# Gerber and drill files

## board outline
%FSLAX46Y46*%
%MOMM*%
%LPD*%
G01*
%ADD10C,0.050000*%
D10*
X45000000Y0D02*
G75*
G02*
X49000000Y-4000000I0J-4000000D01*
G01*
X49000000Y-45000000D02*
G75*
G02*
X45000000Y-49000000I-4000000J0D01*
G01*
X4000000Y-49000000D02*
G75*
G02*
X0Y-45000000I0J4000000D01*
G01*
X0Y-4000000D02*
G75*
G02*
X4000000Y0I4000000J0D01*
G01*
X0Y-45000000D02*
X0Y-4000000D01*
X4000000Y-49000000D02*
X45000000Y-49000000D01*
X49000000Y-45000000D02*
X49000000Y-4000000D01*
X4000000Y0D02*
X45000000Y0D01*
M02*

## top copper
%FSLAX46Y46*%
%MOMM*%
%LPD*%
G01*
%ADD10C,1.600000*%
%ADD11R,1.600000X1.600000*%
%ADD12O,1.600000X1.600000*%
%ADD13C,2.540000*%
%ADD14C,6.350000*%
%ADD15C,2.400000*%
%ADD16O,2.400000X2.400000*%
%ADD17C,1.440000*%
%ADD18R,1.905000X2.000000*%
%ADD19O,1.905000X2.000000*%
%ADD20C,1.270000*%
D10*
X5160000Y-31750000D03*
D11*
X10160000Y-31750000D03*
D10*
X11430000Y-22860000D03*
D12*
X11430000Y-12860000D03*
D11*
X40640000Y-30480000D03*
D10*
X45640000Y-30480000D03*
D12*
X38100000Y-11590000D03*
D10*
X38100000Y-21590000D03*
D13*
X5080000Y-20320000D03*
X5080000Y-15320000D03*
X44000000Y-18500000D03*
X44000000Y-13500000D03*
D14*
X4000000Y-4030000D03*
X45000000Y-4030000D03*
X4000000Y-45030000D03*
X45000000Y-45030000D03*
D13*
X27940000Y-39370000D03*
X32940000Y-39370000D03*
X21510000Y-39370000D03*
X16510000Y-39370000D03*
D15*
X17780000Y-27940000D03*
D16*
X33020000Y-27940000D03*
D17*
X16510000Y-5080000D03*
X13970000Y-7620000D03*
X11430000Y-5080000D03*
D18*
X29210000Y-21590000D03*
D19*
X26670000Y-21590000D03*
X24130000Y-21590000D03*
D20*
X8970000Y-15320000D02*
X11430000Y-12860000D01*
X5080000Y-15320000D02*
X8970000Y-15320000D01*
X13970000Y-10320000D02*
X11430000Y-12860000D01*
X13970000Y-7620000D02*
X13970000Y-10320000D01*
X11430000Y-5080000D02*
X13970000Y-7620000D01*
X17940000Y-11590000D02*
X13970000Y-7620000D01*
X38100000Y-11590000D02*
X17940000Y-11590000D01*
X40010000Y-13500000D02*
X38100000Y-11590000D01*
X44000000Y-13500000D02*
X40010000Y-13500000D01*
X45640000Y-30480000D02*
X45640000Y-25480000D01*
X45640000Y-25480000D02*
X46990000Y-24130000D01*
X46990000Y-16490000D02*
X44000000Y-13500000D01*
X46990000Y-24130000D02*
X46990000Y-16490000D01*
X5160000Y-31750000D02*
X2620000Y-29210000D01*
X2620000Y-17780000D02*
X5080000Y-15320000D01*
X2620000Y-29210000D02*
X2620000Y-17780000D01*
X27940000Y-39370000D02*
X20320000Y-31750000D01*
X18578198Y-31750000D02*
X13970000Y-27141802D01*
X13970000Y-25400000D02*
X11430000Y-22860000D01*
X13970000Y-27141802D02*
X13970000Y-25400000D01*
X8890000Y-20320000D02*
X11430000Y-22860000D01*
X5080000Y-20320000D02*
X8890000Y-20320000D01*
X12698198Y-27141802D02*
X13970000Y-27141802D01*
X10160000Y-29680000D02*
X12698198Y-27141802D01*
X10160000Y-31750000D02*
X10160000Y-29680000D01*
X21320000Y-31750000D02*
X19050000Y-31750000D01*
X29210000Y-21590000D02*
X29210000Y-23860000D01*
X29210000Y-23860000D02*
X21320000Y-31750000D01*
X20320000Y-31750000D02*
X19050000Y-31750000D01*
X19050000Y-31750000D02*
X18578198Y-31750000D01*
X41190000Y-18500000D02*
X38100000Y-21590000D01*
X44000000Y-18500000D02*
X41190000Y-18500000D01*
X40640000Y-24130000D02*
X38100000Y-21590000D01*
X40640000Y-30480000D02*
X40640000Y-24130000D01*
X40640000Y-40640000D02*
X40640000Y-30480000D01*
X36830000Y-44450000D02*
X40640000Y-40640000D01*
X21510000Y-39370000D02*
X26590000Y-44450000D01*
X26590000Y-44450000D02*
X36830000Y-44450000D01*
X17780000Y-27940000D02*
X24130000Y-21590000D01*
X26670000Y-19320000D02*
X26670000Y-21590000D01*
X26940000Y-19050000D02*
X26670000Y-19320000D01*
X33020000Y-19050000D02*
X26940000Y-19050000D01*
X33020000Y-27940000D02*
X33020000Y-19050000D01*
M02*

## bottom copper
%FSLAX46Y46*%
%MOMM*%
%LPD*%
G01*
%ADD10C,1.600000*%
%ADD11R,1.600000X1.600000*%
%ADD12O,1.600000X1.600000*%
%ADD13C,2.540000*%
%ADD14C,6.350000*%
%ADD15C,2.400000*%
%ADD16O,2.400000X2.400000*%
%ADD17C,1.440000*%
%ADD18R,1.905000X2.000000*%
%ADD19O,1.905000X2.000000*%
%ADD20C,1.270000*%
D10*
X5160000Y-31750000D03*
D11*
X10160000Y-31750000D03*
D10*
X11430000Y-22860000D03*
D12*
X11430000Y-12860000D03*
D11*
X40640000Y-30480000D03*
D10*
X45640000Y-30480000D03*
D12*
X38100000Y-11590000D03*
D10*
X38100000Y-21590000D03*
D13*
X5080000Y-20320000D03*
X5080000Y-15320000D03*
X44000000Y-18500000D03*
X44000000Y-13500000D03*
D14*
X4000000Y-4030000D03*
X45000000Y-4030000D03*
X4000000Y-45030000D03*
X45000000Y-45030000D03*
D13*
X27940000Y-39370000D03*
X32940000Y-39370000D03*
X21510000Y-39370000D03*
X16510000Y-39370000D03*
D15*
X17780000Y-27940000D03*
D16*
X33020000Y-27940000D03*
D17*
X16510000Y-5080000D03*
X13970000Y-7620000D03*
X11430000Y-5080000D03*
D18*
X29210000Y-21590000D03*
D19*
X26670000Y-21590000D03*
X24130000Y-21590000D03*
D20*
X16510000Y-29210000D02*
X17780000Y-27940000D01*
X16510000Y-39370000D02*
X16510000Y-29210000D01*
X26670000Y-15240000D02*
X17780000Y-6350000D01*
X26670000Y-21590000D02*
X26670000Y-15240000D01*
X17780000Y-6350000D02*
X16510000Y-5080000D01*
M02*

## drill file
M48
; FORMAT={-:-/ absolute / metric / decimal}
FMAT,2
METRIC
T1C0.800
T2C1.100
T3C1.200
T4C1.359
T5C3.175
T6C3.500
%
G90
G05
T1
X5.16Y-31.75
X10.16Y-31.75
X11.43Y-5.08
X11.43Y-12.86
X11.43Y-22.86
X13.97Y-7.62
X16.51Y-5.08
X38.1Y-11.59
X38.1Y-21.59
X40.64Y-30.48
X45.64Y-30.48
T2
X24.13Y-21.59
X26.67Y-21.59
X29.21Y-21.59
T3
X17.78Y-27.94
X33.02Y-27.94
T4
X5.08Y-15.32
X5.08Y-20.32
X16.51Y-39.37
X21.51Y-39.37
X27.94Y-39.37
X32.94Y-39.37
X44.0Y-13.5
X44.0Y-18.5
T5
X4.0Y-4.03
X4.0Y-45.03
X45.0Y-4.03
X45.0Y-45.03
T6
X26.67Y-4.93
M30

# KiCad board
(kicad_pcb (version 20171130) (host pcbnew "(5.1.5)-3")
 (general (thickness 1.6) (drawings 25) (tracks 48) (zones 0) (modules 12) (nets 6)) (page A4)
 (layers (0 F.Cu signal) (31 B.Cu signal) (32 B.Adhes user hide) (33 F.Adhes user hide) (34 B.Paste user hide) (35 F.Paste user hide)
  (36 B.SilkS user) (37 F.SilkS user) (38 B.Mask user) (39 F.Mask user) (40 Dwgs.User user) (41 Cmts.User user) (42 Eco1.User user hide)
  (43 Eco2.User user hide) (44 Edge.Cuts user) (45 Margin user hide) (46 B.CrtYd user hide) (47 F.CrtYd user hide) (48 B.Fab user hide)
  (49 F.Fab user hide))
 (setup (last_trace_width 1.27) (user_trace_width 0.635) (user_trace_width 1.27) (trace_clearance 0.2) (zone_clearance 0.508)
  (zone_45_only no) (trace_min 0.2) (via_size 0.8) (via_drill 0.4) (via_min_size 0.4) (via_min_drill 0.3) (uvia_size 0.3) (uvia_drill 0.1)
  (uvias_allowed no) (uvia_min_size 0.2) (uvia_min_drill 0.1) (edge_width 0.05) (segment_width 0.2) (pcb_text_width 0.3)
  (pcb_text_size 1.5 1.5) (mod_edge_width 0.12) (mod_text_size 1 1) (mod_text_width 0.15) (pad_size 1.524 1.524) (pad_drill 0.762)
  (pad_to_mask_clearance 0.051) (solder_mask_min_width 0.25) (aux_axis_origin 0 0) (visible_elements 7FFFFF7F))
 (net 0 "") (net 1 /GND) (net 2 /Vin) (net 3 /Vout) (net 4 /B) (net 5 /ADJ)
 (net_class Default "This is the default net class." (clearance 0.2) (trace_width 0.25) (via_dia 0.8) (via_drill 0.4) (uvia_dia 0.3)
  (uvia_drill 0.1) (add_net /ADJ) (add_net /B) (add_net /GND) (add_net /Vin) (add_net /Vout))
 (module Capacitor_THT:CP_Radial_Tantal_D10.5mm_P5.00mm (layer F.Cu) (at 10.16 31.75 180)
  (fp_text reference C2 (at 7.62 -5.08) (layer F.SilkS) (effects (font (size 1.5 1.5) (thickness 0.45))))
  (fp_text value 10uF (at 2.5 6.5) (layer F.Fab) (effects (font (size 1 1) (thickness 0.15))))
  (pad 2 thru_hole circle (at 5 0 180) (size 1.6 1.6) (drill 0.8) (layers *.Cu *.Mask) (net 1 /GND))
  (pad 1 thru_hole rect (at 0 0 180) (size 1.6 1.6) (drill 0.8) (layers *.Cu *.Mask) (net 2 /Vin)))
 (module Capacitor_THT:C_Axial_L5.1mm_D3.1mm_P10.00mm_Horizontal (layer F.Cu) (at 11.43 22.86 90)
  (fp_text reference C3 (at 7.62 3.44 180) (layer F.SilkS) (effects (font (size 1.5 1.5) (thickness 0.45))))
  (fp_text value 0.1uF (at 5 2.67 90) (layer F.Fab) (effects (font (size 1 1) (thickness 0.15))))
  (pad 1 thru_hole circle (at 0 0 90) (size 1.6 1.6) (drill 0.8) (layers *.Cu *.Mask) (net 2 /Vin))
  (pad 2 thru_hole oval (at 10 0 90) (size 1.6 1.6) (drill 0.8) (layers *.Cu *.Mask) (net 1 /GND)))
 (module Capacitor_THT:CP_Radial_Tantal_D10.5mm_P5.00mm (layer F.Cu) (at 40.64 30.48)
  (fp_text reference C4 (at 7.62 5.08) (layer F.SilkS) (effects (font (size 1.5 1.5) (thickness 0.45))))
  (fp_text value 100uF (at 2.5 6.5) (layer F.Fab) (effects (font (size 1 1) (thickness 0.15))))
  (pad 1 thru_hole rect (at 0 0) (size 1.6 1.6) (drill 0.8) (layers *.Cu *.Mask) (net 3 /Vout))
  (pad 2 thru_hole circle (at 5 0) (size 1.6 1.6) (drill 0.8) (layers *.Cu *.Mask) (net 1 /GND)))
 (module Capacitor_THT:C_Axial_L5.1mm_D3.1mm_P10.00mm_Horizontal (layer F.Cu) (at 38.1 21.59 90)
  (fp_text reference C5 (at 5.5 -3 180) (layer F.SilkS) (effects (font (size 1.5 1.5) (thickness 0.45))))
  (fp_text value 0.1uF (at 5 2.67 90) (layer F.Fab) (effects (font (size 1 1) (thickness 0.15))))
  (pad 2 thru_hole oval (at 10 0 90) (size 1.6 1.6) (drill 0.8) (layers *.Cu *.Mask) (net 1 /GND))
  (pad 1 thru_hole circle (at 0 0 90) (size 1.6 1.6) (drill 0.8) (layers *.Cu *.Mask) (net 3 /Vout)))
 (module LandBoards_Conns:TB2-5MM (layer F.Cu) (at 5.08 20.32 90)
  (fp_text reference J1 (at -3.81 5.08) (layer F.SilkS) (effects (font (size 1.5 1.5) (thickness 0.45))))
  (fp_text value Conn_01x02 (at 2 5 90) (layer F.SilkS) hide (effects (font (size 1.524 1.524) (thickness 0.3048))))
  (pad 1 thru_hole circle (at 0 0 90) (size 2.54 2.54) (drill 1.3589) (layers *.Cu *.Mask F.SilkS) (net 2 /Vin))
  (pad 2 thru_hole circle (at 5 0 90) (size 2.54 2.54) (drill 1.3589) (layers *.Cu *.Mask F.SilkS) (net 1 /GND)))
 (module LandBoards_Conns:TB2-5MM (layer F.Cu) (at 44 13.5 270)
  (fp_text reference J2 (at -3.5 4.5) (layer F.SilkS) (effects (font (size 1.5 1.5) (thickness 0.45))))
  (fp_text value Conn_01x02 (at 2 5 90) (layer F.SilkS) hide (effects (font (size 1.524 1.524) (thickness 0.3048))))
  (pad 2 thru_hole circle (at 5 0 270) (size 2.54 2.54) (drill 1.3589) (layers *.Cu *.Mask F.SilkS) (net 3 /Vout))
  (pad 1 thru_hole circle (at 0 0 270) (size 2.54 2.54) (drill 1.3589) (layers *.Cu *.Mask F.SilkS) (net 1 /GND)))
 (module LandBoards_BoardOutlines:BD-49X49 (layer F.Cu) (at 0 49.03)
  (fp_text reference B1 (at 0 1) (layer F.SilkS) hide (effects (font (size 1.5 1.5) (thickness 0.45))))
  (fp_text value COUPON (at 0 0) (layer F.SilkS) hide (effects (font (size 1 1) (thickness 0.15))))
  (pad 1 thru_hole circle (at 4 -45) (size 6.35 6.35) (drill 3.175) (layers *.Cu *.Mask F.SilkS))
  (pad 2 thru_hole circle (at 45 -45) (size 6.35 6.35) (drill 3.175) (layers *.Cu *.Mask F.SilkS))
  (pad 3 thru_hole circle (at 4 -4) (size 6.35 6.35) (drill 3.175) (layers *.Cu *.Mask F.SilkS))
  (pad 4 thru_hole circle (at 45 -4) (size 6.35 6.35) (drill 3.175) (layers *.Cu *.Mask F.SilkS)))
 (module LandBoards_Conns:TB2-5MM (layer F.Cu) (at 27.94 39.37)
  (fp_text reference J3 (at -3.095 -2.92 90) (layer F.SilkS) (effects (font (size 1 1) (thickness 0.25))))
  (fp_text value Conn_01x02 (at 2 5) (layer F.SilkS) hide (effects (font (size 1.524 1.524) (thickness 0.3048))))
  (pad 1 thru_hole circle (at 0 0) (size 2.54 2.54) (drill 1.3589) (layers *.Cu *.Mask F.SilkS) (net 2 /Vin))
  (pad 2 thru_hole circle (at 5 0) (size 2.54 2.54) (drill 1.3589) (layers *.Cu *.Mask F.SilkS)))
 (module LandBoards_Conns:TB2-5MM (layer F.Cu) (at 16.51 39.37)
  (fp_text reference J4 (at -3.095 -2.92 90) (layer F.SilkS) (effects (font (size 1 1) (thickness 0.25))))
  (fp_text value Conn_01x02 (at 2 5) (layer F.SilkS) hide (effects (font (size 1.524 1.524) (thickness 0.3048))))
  (pad 2 thru_hole circle (at 5 0) (size 2.54 2.54) (drill 1.3589) (layers *.Cu *.Mask F.SilkS) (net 3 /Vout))
  (pad 1 thru_hole circle (at 0 0) (size 2.54 2.54) (drill 1.3589) (layers *.Cu *.Mask F.SilkS) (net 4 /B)))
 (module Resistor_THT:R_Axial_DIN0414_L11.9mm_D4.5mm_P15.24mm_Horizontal (layer F.Cu) (at 17.78 27.94)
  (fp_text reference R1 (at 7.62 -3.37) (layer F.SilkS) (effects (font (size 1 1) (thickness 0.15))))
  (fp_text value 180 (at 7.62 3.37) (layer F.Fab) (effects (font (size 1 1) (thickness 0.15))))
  (pad 1 thru_hole circle (at 0 0) (size 2.4 2.4) (drill 1.2) (layers *.Cu *.Mask) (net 4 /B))
  (pad 2 thru_hole oval (at 15.24 0) (size 2.4 2.4) (drill 1.2) (layers *.Cu *.Mask) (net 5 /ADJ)))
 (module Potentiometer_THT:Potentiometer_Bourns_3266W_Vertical (layer F.Cu) (at 16.51 5.08)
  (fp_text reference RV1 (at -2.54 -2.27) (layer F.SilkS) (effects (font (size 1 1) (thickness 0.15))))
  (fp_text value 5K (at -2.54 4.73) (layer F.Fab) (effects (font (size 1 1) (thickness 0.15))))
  (pad 1 thru_hole circle (at 0 0) (size 1.44 1.44) (drill 0.8) (layers *.Cu *.Mask) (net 5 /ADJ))
  (pad 2 thru_hole circle (at -2.54 2.54) (size 1.44 1.44) (drill 0.8) (layers *.Cu *.Mask) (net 1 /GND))
  (pad 3 thru_hole circle (at -5.08 0) (size 1.44 1.44) (drill 0.8) (layers *.Cu *.Mask) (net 1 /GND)))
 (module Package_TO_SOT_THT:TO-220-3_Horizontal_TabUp (layer F.Cu) (at 29.21 21.59 180)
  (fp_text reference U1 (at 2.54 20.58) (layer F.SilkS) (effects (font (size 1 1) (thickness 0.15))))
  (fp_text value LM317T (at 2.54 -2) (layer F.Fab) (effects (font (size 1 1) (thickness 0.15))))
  (pad "" np_thru_hole oval (at 2.54 16.66 180) (size 3.5 3.5) (drill 3.5) (layers *.Cu *.Mask))
  (pad 1 thru_hole rect (at 0 0 180) (size 1.905 2) (drill 1.1) (layers *.Cu *.Mask) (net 2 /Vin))
  (pad 2 thru_hole oval (at 2.54 0 180) (size 1.905 2) (drill 1.1) (layers *.Cu *.Mask) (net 5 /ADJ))
  (pad 3 thru_hole oval (at 5.08 0 180) (size 1.905 2) (drill 1.1) (layers *.Cu *.Mask) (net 4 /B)))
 (gr_arc (start 45 4) (end 49 4) (angle -90) (layer Edge.Cuts) (width 0.05))
 (gr_arc (start 45 45) (end 45 49) (angle -90) (layer Edge.Cuts) (width 0.05))
 (gr_arc (start 4 45) (end 0 45) (angle -90) (layer Edge.Cuts) (width 0.05))
 (gr_arc (start 4 4) (end 4 0) (angle -90) (layer Edge.Cuts) (width 0.05))
 (gr_line (start 0 45) (end 0 4) (layer Edge.Cuts) (width 0.05))
 (gr_line (start 4 49) (end 45 49) (layer Edge.Cuts) (width 0.05))
 (gr_line (start 49 45) (end 49 4) (layer Edge.Cuts) (width 0.05))
 (gr_line (start 4 0) (end 45 0) (layer Edge.Cuts) (width 0.05))
 (segment (start 8.97 15.32) (end 11.43 12.86) (width 1.27) (layer F.Cu) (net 1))
 (segment (start 5.08 15.32) (end 8.97 15.32) (width 1.27) (layer F.Cu) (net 1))
 (segment (start 13.97 10.32) (end 11.43 12.86) (width 1.27) (layer F.Cu) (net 1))
 (segment (start 13.97 7.62) (end 13.97 10.32) (width 1.27) (layer F.Cu) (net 1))
 (segment (start 11.43 5.08) (end 13.97 7.62) (width 1.27) (layer F.Cu) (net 1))
 (segment (start 17.94 11.59) (end 13.97 7.62) (width 1.27) (layer F.Cu) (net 1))
 (segment (start 38.1 11.59) (end 17.94 11.59) (width 1.27) (layer F.Cu) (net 1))
 (segment (start 40.01 13.5) (end 38.1 11.59) (width 1.27) (layer F.Cu) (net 1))
 (segment (start 44 13.5) (end 40.01 13.5) (width 1.27) (layer F.Cu) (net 1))
 (segment (start 45.64 30.48) (end 45.64 25.48) (width 1.27) (layer F.Cu) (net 1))
 (segment (start 45.64 25.48) (end 46.99 24.13) (width 1.27) (layer F.Cu) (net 1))
 (segment (start 46.99 16.49) (end 44 13.5) (width 1.27) (layer F.Cu) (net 1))
 (segment (start 46.99 24.13) (end 46.99 16.49) (width 1.27) (layer F.Cu) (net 1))
 (segment (start 5.16 31.75) (end 2.62 29.21) (width 1.27) (layer F.Cu) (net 1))
 (segment (start 2.62 17.78) (end 5.08 15.32) (width 1.27) (layer F.Cu) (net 1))
 (segment (start 2.62 29.21) (end 2.62 17.78) (width 1.27) (layer F.Cu) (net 1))
 (segment (start 27.94 39.37) (end 20.32 31.75) (width 1.27) (layer F.Cu) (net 2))
 (segment (start 18.578198 31.75) (end 13.97 27.141802) (width 1.27) (layer F.Cu) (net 2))
 (segment (start 13.97 25.4) (end 11.43 22.86) (width 1.27) (layer F.Cu) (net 2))
 (segment (start 13.97 27.141802) (end 13.97 25.4) (width 1.27) (layer F.Cu) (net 2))
 (segment (start 8.89 20.32) (end 11.43 22.86) (width 1.27) (layer F.Cu) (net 2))
 (segment (start 5.08 20.32) (end 8.89 20.32) (width 1.27) (layer F.Cu) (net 2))
 (segment (start 12.698198 27.141802) (end 13.97 27.141802) (width 1.27) (layer F.Cu) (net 2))
 (segment (start 10.16 29.68) (end 12.698198 27.141802) (width 1.27) (layer F.Cu) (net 2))
 (segment (start 10.16 31.75) (end 10.16 29.68) (width 1.27) (layer F.Cu) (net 2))
 (segment (start 21.32 31.75) (end 19.05 31.75) (width 1.27) (layer F.Cu) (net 2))
 (segment (start 29.21 21.59) (end 29.21 23.86) (width 1.27) (layer F.Cu) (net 2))
 (segment (start 29.21 23.86) (end 21.32 31.75) (width 1.27) (layer F.Cu) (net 2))
 (segment (start 20.32 31.75) (end 19.05 31.75) (width 1.27) (layer F.Cu) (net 2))
 (segment (start 19.05 31.75) (end 18.578198 31.75) (width 1.27) (layer F.Cu) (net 2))
 (segment (start 41.19 18.5) (end 38.1 21.59) (width 1.27) (layer F.Cu) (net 3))
 (segment (start 44 18.5) (end 41.19 18.5) (width 1.27) (layer F.Cu) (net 3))
 (segment (start 40.64 24.13) (end 38.1 21.59) (width 1.27) (layer F.Cu) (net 3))
 (segment (start 40.64 30.48) (end 40.64 24.13) (width 1.27) (layer F.Cu) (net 3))
 (segment (start 40.64 40.64) (end 40.64 30.48) (width 1.27) (layer F.Cu) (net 3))
 (segment (start 36.83 44.45) (end 40.64 40.64) (width 1.27) (layer F.Cu) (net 3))
 (segment (start 21.51 39.37) (end 26.59 44.45) (width 1.27) (layer F.Cu) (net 3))
 (segment (start 26.59 44.45) (end 36.83 44.45) (width 1.27) (layer F.Cu) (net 3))
 (segment (start 17.78 27.94) (end 24.13 21.59) (width 1.27) (layer F.Cu) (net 4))
 (segment (start 16.51 29.21) (end 17.78 27.94) (width 1.27) (layer B.Cu) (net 4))
 (segment (start 16.51 39.37) (end 16.51 29.21) (width 1.27) (layer B.Cu) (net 4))
 (segment (start 26.67 19.32) (end 26.67 21.59) (width 1.27) (layer F.Cu) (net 5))
 (segment (start 26.94 19.05) (end 26.67 19.32) (width 1.27) (layer F.Cu) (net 5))
 (segment (start 33.02 19.05) (end 26.94 19.05) (width 1.27) (layer F.Cu) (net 5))
 (segment (start 33.02 27.94) (end 33.02 19.05) (width 1.27) (layer F.Cu) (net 5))
 (segment (start 26.67 15.24) (end 17.78 6.35) (width 1.27) (layer B.Cu) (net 5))
 (segment (start 26.67 21.59) (end 26.67 15.24) (width 1.27) (layer B.Cu) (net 5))
 (segment (start 17.78 6.35) (end 16.51 5.08) (width 1.27) (layer B.Cu) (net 5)))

